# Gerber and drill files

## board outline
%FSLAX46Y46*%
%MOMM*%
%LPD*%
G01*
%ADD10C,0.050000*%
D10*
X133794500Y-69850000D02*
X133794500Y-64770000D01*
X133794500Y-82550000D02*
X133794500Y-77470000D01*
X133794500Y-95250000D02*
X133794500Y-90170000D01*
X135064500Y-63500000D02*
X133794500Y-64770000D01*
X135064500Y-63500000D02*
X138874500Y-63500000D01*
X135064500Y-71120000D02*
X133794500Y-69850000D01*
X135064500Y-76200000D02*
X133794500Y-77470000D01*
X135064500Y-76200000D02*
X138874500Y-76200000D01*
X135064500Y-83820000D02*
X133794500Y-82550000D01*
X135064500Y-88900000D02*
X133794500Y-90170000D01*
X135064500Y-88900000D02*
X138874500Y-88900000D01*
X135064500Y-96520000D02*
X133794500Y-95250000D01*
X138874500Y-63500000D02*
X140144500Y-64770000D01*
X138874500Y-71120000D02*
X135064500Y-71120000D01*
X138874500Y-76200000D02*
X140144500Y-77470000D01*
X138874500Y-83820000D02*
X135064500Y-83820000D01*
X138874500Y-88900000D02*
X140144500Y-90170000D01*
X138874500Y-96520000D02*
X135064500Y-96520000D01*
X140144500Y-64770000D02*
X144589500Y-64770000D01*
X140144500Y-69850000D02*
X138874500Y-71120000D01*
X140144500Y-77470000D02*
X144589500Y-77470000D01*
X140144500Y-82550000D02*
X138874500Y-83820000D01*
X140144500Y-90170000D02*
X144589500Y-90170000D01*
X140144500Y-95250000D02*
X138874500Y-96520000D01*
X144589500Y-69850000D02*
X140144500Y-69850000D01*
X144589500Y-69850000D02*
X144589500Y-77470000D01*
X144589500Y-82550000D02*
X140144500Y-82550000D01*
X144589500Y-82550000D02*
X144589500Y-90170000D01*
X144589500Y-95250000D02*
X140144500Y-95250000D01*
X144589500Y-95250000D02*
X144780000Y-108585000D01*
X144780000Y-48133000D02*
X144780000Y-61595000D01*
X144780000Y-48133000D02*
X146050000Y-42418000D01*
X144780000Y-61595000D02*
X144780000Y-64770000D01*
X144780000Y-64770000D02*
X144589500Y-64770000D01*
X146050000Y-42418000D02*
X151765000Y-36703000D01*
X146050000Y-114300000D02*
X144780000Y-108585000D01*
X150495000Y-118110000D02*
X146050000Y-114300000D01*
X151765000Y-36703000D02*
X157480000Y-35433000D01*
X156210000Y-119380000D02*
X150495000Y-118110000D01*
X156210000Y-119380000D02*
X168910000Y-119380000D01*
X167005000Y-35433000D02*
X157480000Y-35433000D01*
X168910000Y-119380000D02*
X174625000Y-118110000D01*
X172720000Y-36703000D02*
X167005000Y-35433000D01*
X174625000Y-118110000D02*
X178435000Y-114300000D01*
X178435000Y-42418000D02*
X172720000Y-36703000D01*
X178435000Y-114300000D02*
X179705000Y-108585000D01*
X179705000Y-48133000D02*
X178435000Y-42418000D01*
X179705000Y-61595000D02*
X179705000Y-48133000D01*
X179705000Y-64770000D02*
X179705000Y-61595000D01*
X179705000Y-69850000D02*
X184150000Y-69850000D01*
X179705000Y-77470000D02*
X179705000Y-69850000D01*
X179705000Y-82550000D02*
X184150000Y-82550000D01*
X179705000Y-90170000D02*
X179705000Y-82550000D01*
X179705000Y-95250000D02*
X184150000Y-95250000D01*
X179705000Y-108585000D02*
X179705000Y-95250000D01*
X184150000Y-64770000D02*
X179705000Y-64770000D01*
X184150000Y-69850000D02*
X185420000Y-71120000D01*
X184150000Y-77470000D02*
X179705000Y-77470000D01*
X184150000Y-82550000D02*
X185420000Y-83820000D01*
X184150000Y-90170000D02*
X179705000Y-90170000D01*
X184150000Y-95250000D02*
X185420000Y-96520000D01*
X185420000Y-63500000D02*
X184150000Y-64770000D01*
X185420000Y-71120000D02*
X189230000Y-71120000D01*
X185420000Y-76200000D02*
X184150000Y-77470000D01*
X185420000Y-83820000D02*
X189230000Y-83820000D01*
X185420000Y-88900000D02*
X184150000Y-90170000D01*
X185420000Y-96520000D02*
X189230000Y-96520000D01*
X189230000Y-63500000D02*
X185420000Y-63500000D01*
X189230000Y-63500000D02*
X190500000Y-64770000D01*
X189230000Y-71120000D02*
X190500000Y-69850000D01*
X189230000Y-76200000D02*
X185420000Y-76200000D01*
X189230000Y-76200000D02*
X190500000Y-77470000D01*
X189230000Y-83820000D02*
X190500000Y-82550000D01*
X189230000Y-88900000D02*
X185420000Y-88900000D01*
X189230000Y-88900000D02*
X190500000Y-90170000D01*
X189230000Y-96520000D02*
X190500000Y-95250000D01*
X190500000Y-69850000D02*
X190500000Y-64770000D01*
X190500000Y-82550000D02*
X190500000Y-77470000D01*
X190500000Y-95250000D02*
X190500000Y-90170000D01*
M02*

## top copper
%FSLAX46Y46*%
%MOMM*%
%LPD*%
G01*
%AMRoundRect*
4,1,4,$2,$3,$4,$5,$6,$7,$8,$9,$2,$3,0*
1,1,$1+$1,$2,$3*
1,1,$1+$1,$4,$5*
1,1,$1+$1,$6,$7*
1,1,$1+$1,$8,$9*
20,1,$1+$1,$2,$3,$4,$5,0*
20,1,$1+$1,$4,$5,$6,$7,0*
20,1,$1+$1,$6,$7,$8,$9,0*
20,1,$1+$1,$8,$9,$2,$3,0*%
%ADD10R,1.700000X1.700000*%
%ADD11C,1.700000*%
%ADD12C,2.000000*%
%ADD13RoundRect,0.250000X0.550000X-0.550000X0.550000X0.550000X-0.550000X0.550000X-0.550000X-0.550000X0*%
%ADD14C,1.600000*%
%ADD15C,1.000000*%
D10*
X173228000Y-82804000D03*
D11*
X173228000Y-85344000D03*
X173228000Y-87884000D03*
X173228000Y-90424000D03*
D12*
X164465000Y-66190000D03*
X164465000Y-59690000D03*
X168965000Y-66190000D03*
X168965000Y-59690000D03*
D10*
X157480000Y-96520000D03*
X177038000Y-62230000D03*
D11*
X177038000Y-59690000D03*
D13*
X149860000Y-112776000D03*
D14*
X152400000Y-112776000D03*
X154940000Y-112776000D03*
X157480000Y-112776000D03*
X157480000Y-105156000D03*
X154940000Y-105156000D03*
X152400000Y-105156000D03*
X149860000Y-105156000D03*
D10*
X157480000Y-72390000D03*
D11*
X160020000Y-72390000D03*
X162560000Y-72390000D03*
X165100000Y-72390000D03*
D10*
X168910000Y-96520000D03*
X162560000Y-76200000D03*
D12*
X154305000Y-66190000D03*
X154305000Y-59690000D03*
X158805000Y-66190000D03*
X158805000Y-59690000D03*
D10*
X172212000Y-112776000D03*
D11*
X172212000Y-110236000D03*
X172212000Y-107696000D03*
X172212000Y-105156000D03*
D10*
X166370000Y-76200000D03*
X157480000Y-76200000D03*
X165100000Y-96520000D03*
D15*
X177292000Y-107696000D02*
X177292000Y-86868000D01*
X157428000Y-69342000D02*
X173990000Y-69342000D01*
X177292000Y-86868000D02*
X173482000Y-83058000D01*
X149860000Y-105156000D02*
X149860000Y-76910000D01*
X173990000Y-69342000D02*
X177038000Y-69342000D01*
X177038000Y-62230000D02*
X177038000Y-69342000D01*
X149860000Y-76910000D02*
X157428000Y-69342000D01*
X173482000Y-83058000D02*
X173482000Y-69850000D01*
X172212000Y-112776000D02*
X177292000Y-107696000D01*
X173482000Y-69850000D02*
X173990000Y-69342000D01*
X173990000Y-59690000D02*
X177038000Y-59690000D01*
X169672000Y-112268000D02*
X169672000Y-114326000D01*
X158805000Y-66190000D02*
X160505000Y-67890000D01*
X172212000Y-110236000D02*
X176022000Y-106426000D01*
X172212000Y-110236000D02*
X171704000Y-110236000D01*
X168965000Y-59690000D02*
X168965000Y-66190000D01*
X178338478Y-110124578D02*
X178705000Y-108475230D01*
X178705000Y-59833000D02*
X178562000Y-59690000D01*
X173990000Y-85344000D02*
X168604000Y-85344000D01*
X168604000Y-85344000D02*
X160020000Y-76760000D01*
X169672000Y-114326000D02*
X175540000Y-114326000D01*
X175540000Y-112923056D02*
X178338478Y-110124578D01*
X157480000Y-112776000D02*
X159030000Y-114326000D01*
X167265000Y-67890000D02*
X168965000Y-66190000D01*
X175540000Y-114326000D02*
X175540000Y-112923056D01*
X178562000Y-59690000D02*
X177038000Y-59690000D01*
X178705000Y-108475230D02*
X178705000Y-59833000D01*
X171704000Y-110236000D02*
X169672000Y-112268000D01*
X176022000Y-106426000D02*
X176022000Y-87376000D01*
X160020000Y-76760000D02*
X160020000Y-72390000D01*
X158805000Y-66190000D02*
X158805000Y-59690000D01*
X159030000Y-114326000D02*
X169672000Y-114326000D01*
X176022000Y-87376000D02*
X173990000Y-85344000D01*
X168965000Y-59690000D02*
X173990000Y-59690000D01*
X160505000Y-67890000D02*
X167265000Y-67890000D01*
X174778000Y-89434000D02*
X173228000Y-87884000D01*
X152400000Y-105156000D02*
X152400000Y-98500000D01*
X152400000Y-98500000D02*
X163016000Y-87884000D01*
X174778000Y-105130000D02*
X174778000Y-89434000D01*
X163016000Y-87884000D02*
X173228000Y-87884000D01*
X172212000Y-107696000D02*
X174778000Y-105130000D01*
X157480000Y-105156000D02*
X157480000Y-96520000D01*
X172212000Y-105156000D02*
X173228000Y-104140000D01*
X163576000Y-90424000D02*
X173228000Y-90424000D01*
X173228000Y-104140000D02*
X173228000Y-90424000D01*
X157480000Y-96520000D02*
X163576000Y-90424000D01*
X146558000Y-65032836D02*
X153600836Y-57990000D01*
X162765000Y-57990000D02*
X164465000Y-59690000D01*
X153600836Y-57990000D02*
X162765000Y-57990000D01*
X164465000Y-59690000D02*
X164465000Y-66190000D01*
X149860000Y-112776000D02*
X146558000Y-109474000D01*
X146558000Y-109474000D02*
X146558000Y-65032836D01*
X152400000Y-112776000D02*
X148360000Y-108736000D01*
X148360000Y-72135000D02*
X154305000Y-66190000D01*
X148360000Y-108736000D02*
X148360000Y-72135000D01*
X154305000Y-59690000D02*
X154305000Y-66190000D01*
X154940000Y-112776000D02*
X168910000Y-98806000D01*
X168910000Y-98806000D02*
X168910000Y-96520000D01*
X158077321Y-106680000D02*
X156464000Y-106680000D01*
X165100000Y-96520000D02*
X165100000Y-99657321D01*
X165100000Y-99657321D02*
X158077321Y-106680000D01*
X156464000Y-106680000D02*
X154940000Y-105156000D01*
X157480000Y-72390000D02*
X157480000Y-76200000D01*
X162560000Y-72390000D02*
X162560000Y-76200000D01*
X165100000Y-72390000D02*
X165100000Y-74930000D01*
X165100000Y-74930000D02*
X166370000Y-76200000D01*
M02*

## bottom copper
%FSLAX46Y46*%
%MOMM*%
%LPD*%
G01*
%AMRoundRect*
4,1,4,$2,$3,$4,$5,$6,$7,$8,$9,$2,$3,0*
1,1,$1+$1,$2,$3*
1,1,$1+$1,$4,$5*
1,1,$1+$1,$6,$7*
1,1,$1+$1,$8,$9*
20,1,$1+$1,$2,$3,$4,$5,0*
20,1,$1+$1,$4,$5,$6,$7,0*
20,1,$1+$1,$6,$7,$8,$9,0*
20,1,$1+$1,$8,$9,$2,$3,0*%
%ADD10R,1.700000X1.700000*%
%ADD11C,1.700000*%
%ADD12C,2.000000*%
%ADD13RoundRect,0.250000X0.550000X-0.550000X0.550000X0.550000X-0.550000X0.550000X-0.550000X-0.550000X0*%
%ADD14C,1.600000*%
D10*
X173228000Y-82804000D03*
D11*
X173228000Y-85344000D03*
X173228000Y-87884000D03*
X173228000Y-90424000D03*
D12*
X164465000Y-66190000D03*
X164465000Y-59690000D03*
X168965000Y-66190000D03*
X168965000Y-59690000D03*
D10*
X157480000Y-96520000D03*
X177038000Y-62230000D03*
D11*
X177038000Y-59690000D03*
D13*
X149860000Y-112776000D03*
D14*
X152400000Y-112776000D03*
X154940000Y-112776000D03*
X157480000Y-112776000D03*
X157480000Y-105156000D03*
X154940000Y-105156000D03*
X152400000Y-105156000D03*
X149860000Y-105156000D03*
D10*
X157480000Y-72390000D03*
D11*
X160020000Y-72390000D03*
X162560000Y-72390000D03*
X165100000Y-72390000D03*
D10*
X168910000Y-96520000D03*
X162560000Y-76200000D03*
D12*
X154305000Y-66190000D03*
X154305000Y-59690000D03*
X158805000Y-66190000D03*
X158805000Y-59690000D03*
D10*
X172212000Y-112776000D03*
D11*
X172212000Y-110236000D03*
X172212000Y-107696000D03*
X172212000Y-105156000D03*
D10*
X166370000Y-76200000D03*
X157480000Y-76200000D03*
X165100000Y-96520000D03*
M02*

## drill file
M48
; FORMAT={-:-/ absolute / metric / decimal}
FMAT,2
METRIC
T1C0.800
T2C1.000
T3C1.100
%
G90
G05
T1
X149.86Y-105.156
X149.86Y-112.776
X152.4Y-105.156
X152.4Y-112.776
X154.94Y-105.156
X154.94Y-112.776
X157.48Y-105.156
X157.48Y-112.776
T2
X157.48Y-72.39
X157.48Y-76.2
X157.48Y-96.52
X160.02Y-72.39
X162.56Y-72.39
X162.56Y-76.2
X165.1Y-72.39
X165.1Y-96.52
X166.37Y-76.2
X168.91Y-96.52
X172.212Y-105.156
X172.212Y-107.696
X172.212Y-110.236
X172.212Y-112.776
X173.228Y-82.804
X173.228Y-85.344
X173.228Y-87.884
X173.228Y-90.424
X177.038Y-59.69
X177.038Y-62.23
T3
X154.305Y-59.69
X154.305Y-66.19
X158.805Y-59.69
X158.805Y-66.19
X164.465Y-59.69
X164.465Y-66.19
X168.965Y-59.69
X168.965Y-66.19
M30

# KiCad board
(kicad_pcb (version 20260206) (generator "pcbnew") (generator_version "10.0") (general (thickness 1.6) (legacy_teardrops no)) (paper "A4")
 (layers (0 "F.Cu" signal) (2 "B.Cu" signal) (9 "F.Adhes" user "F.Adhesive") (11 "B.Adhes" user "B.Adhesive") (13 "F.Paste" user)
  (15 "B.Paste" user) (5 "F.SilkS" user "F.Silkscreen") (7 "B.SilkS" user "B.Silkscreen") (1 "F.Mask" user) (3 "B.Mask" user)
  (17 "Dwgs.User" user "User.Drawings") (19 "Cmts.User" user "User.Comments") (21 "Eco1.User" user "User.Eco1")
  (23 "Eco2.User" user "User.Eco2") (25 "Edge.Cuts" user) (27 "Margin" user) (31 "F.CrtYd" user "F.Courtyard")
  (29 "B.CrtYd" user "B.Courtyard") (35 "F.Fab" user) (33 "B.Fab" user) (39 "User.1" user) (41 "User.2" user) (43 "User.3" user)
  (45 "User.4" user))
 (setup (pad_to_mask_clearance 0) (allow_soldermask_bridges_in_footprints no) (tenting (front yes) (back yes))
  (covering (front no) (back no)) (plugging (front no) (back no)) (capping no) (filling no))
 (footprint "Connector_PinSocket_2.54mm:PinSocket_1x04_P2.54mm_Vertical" (layer "F.Cu") (at 173.228 82.804)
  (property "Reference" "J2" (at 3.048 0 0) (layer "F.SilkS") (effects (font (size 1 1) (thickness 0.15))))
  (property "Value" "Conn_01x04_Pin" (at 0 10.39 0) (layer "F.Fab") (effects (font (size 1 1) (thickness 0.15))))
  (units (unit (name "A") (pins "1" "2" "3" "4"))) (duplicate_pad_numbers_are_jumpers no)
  (pad "1" thru_hole rect (at 0 0) (size 1.7 1.7) (drill 1) (layers "*.Cu" "*.Mask") (remove_unused_layers no) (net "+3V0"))
  (pad "2" thru_hole circle (at 0 2.54) (size 1.7 1.7) (drill 1) (layers "*.Cu" "*.Mask") (remove_unused_layers no) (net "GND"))
  (pad "3" thru_hole circle (at 0 5.08) (size 1.7 1.7) (drill 1) (layers "*.Cu" "*.Mask") (remove_unused_layers no) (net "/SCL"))
  (pad "4" thru_hole circle (at 0 7.62) (size 1.7 1.7) (drill 1) (layers "*.Cu" "*.Mask") (remove_unused_layers no) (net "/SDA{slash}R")))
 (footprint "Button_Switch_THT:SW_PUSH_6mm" (layer "F.Cu") (at 164.465 66.19 90)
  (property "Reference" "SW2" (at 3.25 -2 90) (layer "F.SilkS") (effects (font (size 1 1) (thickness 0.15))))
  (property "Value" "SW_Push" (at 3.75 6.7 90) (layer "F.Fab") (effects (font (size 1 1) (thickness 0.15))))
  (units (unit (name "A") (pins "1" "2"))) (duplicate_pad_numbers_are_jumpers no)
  (pad "1" thru_hole circle (at 0 0 180) (size 2 2) (drill 1.1) (layers "*.Cu" "*.Mask") (remove_unused_layers no) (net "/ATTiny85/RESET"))
  (pad "1" thru_hole circle (at 6.5 0 180) (size 2 2) (drill 1.1) (layers "*.Cu" "*.Mask") (remove_unused_layers no) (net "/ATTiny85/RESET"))
  (pad "2" thru_hole circle (at 0 4.5 180) (size 2 2) (drill 1.1) (layers "*.Cu" "*.Mask") (remove_unused_layers no) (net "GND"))
  (pad "2" thru_hole circle (at 6.5 4.5 180) (size 2 2) (drill 1.1) (layers "*.Cu" "*.Mask") (remove_unused_layers no) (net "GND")))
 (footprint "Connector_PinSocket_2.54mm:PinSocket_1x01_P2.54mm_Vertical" (layer "F.Cu") (at 157.48 96.52)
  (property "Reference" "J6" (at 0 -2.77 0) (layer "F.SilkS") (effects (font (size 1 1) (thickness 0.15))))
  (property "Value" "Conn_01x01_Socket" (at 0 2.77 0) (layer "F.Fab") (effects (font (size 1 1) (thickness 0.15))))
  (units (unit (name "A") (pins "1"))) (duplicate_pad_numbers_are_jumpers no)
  (pad "1" thru_hole rect (at 0 0) (size 1.7 1.7) (drill 1) (layers "*.Cu" "*.Mask") (remove_unused_layers no) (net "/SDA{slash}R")))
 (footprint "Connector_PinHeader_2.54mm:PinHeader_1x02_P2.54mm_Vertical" (layer "F.Cu") (at 177.038 62.23 180)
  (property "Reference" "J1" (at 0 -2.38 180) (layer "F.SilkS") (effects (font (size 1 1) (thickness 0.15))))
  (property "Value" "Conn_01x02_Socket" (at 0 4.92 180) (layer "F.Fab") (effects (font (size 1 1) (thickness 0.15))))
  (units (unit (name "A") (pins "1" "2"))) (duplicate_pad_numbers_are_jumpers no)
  (pad "1" thru_hole rect (at 0 0 180) (size 1.7 1.7) (drill 1) (layers "*.Cu" "*.Mask") (remove_unused_layers no) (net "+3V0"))
  (pad "2" thru_hole circle (at 0 2.54 180) (size 1.7 1.7) (drill 1) (layers "*.Cu" "*.Mask") (remove_unused_layers no) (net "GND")))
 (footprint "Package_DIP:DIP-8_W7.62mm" (layer "F.Cu") (at 149.86 112.776 90)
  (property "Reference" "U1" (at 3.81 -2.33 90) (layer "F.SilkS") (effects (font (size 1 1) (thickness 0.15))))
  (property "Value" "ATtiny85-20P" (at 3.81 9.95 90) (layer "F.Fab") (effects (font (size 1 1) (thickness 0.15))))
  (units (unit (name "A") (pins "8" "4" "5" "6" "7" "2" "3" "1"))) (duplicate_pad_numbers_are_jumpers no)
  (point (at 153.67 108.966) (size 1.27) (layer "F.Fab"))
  (pad "1" thru_hole roundrect (at 0 0 90) (size 1.6 1.6) (drill 0.8) (layers "*.Cu" "*.Mask") (remove_unused_layers no)
   (roundrect_rratio 0.15625) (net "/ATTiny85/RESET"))
  (pad "2" thru_hole circle (at 0 2.54 90) (size 1.6 1.6) (drill 0.8) (layers "*.Cu" "*.Mask") (remove_unused_layers no)
   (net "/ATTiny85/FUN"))
  (pad "3" thru_hole circle (at 0 5.08 90) (size 1.6 1.6) (drill 0.8) (layers "*.Cu" "*.Mask") (remove_unused_layers no) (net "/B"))
  (pad "4" thru_hole circle (at 0 7.62 90) (size 1.6 1.6) (drill 0.8) (layers "*.Cu" "*.Mask") (remove_unused_layers no) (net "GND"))
  (pad "5" thru_hole circle (at 7.62 7.62 90) (size 1.6 1.6) (drill 0.8) (layers "*.Cu" "*.Mask") (remove_unused_layers no)
   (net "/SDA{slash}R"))
  (pad "6" thru_hole circle (at 7.62 5.08 90) (size 1.6 1.6) (drill 0.8) (layers "*.Cu" "*.Mask") (remove_unused_layers no) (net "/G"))
  (pad "7" thru_hole circle (at 7.62 2.54 90) (size 1.6 1.6) (drill 0.8) (layers "*.Cu" "*.Mask") (remove_unused_layers no) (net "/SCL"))
  (pad "8" thru_hole circle (at 7.62 0 90) (size 1.6 1.6) (drill 0.8) (layers "*.Cu" "*.Mask") (remove_unused_layers no) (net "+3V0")))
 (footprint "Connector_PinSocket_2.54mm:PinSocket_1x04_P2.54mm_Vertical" (layer "F.Cu") (at 157.48 72.39 90)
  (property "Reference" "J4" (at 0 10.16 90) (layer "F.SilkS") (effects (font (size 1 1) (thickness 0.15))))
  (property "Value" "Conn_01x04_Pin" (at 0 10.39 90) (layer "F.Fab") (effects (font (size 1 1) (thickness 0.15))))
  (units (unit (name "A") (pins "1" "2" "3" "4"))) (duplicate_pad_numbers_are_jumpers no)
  (pad "1" thru_hole rect (at 0 0 90) (size 1.7 1.7) (drill 1) (layers "*.Cu" "*.Mask") (remove_unused_layers no) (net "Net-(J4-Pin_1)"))
  (pad "2" thru_hole circle (at 0 2.54 90) (size 1.7 1.7) (drill 1) (layers "*.Cu" "*.Mask") (remove_unused_layers no) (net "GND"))
  (pad "3" thru_hole circle (at 0 5.08 90) (size 1.7 1.7) (drill 1) (layers "*.Cu" "*.Mask") (remove_unused_layers no)
   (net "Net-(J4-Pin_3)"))
  (pad "4" thru_hole circle (at 0 7.62 90) (size 1.7 1.7) (drill 1) (layers "*.Cu" "*.Mask") (remove_unused_layers no)
   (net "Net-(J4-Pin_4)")))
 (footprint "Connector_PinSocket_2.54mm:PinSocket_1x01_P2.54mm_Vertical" (layer "F.Cu") (at 168.91 96.52)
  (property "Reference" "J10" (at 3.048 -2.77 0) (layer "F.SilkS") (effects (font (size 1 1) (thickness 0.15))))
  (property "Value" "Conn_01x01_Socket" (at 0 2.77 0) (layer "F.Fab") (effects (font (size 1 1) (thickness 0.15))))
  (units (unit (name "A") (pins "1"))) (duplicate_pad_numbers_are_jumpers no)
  (pad "1" thru_hole rect (at 0 0) (size 1.7 1.7) (drill 1) (layers "*.Cu" "*.Mask") (remove_unused_layers no) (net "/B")))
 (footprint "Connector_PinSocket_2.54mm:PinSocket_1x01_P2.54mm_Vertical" (layer "F.Cu") (at 162.56 76.2)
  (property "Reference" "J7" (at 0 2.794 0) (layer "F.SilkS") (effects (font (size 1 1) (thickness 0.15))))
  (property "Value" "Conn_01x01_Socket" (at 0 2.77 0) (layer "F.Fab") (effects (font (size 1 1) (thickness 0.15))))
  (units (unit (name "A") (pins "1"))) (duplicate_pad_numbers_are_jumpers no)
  (pad "1" thru_hole rect (at 0 0) (size 1.7 1.7) (drill 1) (layers "*.Cu" "*.Mask") (remove_unused_layers no) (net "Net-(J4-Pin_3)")))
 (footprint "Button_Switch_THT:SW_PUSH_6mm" (layer "F.Cu") (at 154.305 66.19 90)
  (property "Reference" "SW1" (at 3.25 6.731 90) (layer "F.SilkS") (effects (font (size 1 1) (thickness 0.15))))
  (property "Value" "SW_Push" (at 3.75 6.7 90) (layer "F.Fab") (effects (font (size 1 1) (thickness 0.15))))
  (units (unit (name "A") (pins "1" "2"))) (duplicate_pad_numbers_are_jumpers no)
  (pad "1" thru_hole circle (at 0 0 180) (size 2 2) (drill 1.1) (layers "*.Cu" "*.Mask") (remove_unused_layers no) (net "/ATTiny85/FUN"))
  (pad "1" thru_hole circle (at 6.5 0 180) (size 2 2) (drill 1.1) (layers "*.Cu" "*.Mask") (remove_unused_layers no) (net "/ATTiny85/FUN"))
  (pad "2" thru_hole circle (at 0 4.5 180) (size 2 2) (drill 1.1) (layers "*.Cu" "*.Mask") (remove_unused_layers no) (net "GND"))
  (pad "2" thru_hole circle (at 6.5 4.5 180) (size 2 2) (drill 1.1) (layers "*.Cu" "*.Mask") (remove_unused_layers no) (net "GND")))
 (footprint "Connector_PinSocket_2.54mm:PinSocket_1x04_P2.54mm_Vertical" (layer "F.Cu") (at 172.212 112.776 180)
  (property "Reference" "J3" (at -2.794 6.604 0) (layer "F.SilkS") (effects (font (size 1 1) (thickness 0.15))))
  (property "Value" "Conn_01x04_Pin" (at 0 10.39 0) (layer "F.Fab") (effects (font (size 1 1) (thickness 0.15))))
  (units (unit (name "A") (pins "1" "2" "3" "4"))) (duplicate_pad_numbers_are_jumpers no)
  (pad "1" thru_hole rect (at 0 0 180) (size 1.7 1.7) (drill 1) (layers "*.Cu" "*.Mask") (remove_unused_layers no) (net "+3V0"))
  (pad "2" thru_hole circle (at 0 2.54 180) (size 1.7 1.7) (drill 1) (layers "*.Cu" "*.Mask") (remove_unused_layers no) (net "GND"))
  (pad "3" thru_hole circle (at 0 5.08 180) (size 1.7 1.7) (drill 1) (layers "*.Cu" "*.Mask") (remove_unused_layers no) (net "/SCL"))
  (pad "4" thru_hole circle (at 0 7.62 180) (size 1.7 1.7) (drill 1) (layers "*.Cu" "*.Mask") (remove_unused_layers no) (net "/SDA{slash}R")))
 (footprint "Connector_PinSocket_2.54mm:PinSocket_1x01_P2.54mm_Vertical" (layer "F.Cu") (at 166.37 76.2)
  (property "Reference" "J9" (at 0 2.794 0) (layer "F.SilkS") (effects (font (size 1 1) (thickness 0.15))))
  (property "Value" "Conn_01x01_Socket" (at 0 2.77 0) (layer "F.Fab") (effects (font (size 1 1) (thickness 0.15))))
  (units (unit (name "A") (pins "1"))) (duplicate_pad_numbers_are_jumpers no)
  (pad "1" thru_hole rect (at 0 0) (size 1.7 1.7) (drill 1) (layers "*.Cu" "*.Mask") (remove_unused_layers no) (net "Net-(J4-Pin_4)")))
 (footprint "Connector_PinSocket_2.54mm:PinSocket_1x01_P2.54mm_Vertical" (layer "F.Cu") (at 157.48 76.2)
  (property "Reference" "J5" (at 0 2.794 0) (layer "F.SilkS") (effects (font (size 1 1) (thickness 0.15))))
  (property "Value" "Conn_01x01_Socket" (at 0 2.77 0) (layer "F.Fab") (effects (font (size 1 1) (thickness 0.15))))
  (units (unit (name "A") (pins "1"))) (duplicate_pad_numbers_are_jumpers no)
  (pad "1" thru_hole rect (at 0 0) (size 1.7 1.7) (drill 1) (layers "*.Cu" "*.Mask") (remove_unused_layers no) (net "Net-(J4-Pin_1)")))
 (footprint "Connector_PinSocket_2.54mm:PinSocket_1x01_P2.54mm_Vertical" (layer "F.Cu") (at 165.1 96.52)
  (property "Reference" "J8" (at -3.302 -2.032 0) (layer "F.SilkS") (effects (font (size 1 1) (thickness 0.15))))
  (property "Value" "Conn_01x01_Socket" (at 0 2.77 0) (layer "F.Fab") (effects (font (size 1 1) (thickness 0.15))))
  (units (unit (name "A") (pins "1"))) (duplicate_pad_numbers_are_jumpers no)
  (pad "1" thru_hole rect (at 0 0) (size 1.7 1.7) (drill 1) (layers "*.Cu" "*.Mask") (remove_unused_layers no) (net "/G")))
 (gr_line (start 133.7945 69.85) (end 133.7945 64.77) (stroke (width 0.05) (type default)) (layer "Edge.Cuts"))
 (gr_line (start 133.7945 82.55) (end 133.7945 77.47) (stroke (width 0.05) (type default)) (layer "Edge.Cuts"))
 (gr_line (start 133.7945 95.25) (end 133.7945 90.17) (stroke (width 0.05) (type default)) (layer "Edge.Cuts"))
 (gr_line (start 135.0645 63.5) (end 133.7945 64.77) (stroke (width 0.05) (type default)) (layer "Edge.Cuts"))
 (gr_line (start 135.0645 63.5) (end 138.8745 63.5) (stroke (width 0.05) (type default)) (layer "Edge.Cuts"))
 (gr_line (start 135.0645 71.12) (end 133.7945 69.85) (stroke (width 0.05) (type default)) (layer "Edge.Cuts"))
 (gr_line (start 135.0645 76.2) (end 133.7945 77.47) (stroke (width 0.05) (type default)) (layer "Edge.Cuts"))
 (gr_line (start 135.0645 76.2) (end 138.8745 76.2) (stroke (width 0.05) (type default)) (layer "Edge.Cuts"))
 (gr_line (start 135.0645 83.82) (end 133.7945 82.55) (stroke (width 0.05) (type default)) (layer "Edge.Cuts"))
 (gr_line (start 135.0645 88.9) (end 133.7945 90.17) (stroke (width 0.05) (type default)) (layer "Edge.Cuts"))
 (gr_line (start 135.0645 88.9) (end 138.8745 88.9) (stroke (width 0.05) (type default)) (layer "Edge.Cuts"))
 (gr_line (start 135.0645 96.52) (end 133.7945 95.25) (stroke (width 0.05) (type default)) (layer "Edge.Cuts"))
 (gr_line (start 138.8745 63.5) (end 140.1445 64.77) (stroke (width 0.05) (type default)) (layer "Edge.Cuts"))
 (gr_line (start 138.8745 71.12) (end 135.0645 71.12) (stroke (width 0.05) (type default)) (layer "Edge.Cuts"))
 (gr_line (start 138.8745 76.2) (end 140.1445 77.47) (stroke (width 0.05) (type default)) (layer "Edge.Cuts"))
 (gr_line (start 138.8745 83.82) (end 135.0645 83.82) (stroke (width 0.05) (type default)) (layer "Edge.Cuts"))
 (gr_line (start 138.8745 88.9) (end 140.1445 90.17) (stroke (width 0.05) (type default)) (layer "Edge.Cuts"))
 (gr_line (start 138.8745 96.52) (end 135.0645 96.52) (stroke (width 0.05) (type default)) (layer "Edge.Cuts"))
 (gr_line (start 140.1445 64.77) (end 144.5895 64.77) (stroke (width 0.05) (type default)) (layer "Edge.Cuts"))
 (gr_line (start 140.1445 69.85) (end 138.8745 71.12) (stroke (width 0.05) (type default)) (layer "Edge.Cuts"))
 (gr_line (start 140.1445 77.47) (end 144.5895 77.47) (stroke (width 0.05) (type default)) (layer "Edge.Cuts"))
 (gr_line (start 140.1445 82.55) (end 138.8745 83.82) (stroke (width 0.05) (type default)) (layer "Edge.Cuts"))
 (gr_line (start 140.1445 90.17) (end 144.5895 90.17) (stroke (width 0.05) (type default)) (layer "Edge.Cuts"))
 (gr_line (start 140.1445 95.25) (end 138.8745 96.52) (stroke (width 0.05) (type default)) (layer "Edge.Cuts"))
 (gr_line (start 144.5895 69.85) (end 140.1445 69.85) (stroke (width 0.05) (type default)) (layer "Edge.Cuts"))
 (gr_line (start 144.5895 69.85) (end 144.5895 77.47) (stroke (width 0.05) (type default)) (layer "Edge.Cuts"))
 (gr_line (start 144.5895 82.55) (end 140.1445 82.55) (stroke (width 0.05) (type default)) (layer "Edge.Cuts"))
 (gr_line (start 144.5895 82.55) (end 144.5895 90.17) (stroke (width 0.05) (type default)) (layer "Edge.Cuts"))
 (gr_line (start 144.5895 95.25) (end 140.1445 95.25) (stroke (width 0.05) (type default)) (layer "Edge.Cuts"))
 (gr_line (start 144.5895 95.25) (end 144.78 108.585) (stroke (width 0.05) (type default)) (layer "Edge.Cuts"))
 (gr_line (start 144.78 48.133) (end 144.78 61.595) (stroke (width 0.05) (type default)) (layer "Edge.Cuts"))
 (gr_line (start 144.78 48.133) (end 146.05 42.418) (stroke (width 0.05) (type default)) (layer "Edge.Cuts"))
 (gr_line (start 144.78 61.595) (end 144.78 64.77) (stroke (width 0.05) (type default)) (layer "Edge.Cuts"))
 (gr_line (start 144.78 64.77) (end 144.5895 64.77) (stroke (width 0.05) (type default)) (layer "Edge.Cuts"))
 (gr_line (start 146.05 42.418) (end 151.765 36.703) (stroke (width 0.05) (type default)) (layer "Edge.Cuts"))
 (gr_line (start 146.05 114.3) (end 144.78 108.585) (stroke (width 0.05) (type default)) (layer "Edge.Cuts"))
 (gr_line (start 150.495 118.11) (end 146.05 114.3) (stroke (width 0.05) (type default)) (layer "Edge.Cuts"))
 (gr_line (start 151.765 36.703) (end 157.48 35.433) (stroke (width 0.05) (type default)) (layer "Edge.Cuts"))
 (gr_line (start 156.21 119.38) (end 150.495 118.11) (stroke (width 0.05) (type default)) (layer "Edge.Cuts"))
 (gr_line (start 156.21 119.38) (end 168.91 119.38) (stroke (width 0.05) (type default)) (layer "Edge.Cuts"))
 (gr_line (start 167.005 35.433) (end 157.48 35.433) (stroke (width 0.05) (type default)) (layer "Edge.Cuts"))
 (gr_line (start 168.91 119.38) (end 174.625 118.11) (stroke (width 0.05) (type default)) (layer "Edge.Cuts"))
 (gr_line (start 172.72 36.703) (end 167.005 35.433) (stroke (width 0.05) (type default)) (layer "Edge.Cuts"))
 (gr_line (start 174.625 118.11) (end 178.435 114.3) (stroke (width 0.05) (type default)) (layer "Edge.Cuts"))
 (gr_line (start 178.435 42.418) (end 172.72 36.703) (stroke (width 0.05) (type default)) (layer "Edge.Cuts"))
 (gr_line (start 178.435 114.3) (end 179.705 108.585) (stroke (width 0.05) (type default)) (layer "Edge.Cuts"))
 (gr_line (start 179.705 48.133) (end 178.435 42.418) (stroke (width 0.05) (type default)) (layer "Edge.Cuts"))
 (gr_line (start 179.705 61.595) (end 179.705 48.133) (stroke (width 0.05) (type default)) (layer "Edge.Cuts"))
 (gr_line (start 179.705 64.77) (end 179.705 61.595) (stroke (width 0.05) (type default)) (layer "Edge.Cuts"))
 (gr_line (start 179.705 69.85) (end 184.15 69.85) (stroke (width 0.05) (type default)) (layer "Edge.Cuts"))
 (gr_line (start 179.705 77.47) (end 179.705 69.85) (stroke (width 0.05) (type default)) (layer "Edge.Cuts"))
 (gr_line (start 179.705 82.55) (end 184.15 82.55) (stroke (width 0.05) (type default)) (layer "Edge.Cuts"))
 (gr_line (start 179.705 90.17) (end 179.705 82.55) (stroke (width 0.05) (type default)) (layer "Edge.Cuts"))
 (gr_line (start 179.705 95.25) (end 184.15 95.25) (stroke (width 0.05) (type default)) (layer "Edge.Cuts"))
 (gr_line (start 179.705 108.585) (end 179.705 95.25) (stroke (width 0.05) (type default)) (layer "Edge.Cuts"))
 (gr_line (start 184.15 64.77) (end 179.705 64.77) (stroke (width 0.05) (type default)) (layer "Edge.Cuts"))
 (gr_line (start 184.15 69.85) (end 185.42 71.12) (stroke (width 0.05) (type default)) (layer "Edge.Cuts"))
 (gr_line (start 184.15 77.47) (end 179.705 77.47) (stroke (width 0.05) (type default)) (layer "Edge.Cuts"))
 (gr_line (start 184.15 82.55) (end 185.42 83.82) (stroke (width 0.05) (type default)) (layer "Edge.Cuts"))
 (gr_line (start 184.15 90.17) (end 179.705 90.17) (stroke (width 0.05) (type default)) (layer "Edge.Cuts"))
 (gr_line (start 184.15 95.25) (end 185.42 96.52) (stroke (width 0.05) (type default)) (layer "Edge.Cuts"))
 (gr_line (start 185.42 63.5) (end 184.15 64.77) (stroke (width 0.05) (type default)) (layer "Edge.Cuts"))
 (gr_line (start 185.42 71.12) (end 189.23 71.12) (stroke (width 0.05) (type default)) (layer "Edge.Cuts"))
 (gr_line (start 185.42 76.2) (end 184.15 77.47) (stroke (width 0.05) (type default)) (layer "Edge.Cuts"))
 (gr_line (start 185.42 83.82) (end 189.23 83.82) (stroke (width 0.05) (type default)) (layer "Edge.Cuts"))
 (gr_line (start 185.42 88.9) (end 184.15 90.17) (stroke (width 0.05) (type default)) (layer "Edge.Cuts"))
 (gr_line (start 185.42 96.52) (end 189.23 96.52) (stroke (width 0.05) (type default)) (layer "Edge.Cuts"))
 (gr_line (start 189.23 63.5) (end 185.42 63.5) (stroke (width 0.05) (type default)) (layer "Edge.Cuts"))
 (gr_line (start 189.23 63.5) (end 190.5 64.77) (stroke (width 0.05) (type default)) (layer "Edge.Cuts"))
 (gr_line (start 189.23 71.12) (end 190.5 69.85) (stroke (width 0.05) (type default)) (layer "Edge.Cuts"))
 (gr_line (start 189.23 76.2) (end 185.42 76.2) (stroke (width 0.05) (type default)) (layer "Edge.Cuts"))
 (gr_line (start 189.23 76.2) (end 190.5 77.47) (stroke (width 0.05) (type default)) (layer "Edge.Cuts"))
 (gr_line (start 189.23 83.82) (end 190.5 82.55) (stroke (width 0.05) (type default)) (layer "Edge.Cuts"))
 (gr_line (start 189.23 88.9) (end 185.42 88.9) (stroke (width 0.05) (type default)) (layer "Edge.Cuts"))
 (gr_line (start 189.23 88.9) (end 190.5 90.17) (stroke (width 0.05) (type default)) (layer "Edge.Cuts"))
 (gr_line (start 189.23 96.52) (end 190.5 95.25) (stroke (width 0.05) (type default)) (layer "Edge.Cuts"))
 (gr_line (start 190.5 69.85) (end 190.5 64.77) (stroke (width 0.05) (type default)) (layer "Edge.Cuts"))
 (gr_line (start 190.5 82.55) (end 190.5 77.47) (stroke (width 0.05) (type default)) (layer "Edge.Cuts"))
 (gr_line (start 190.5 95.25) (end 190.5 90.17) (stroke (width 0.05) (type default)) (layer "Edge.Cuts"))
 (segment (start 177.292 107.696) (end 177.292 86.868) (width 1) (layer "F.Cu") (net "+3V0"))
 (segment (start 157.428 69.342) (end 173.99 69.342) (width 1) (layer "F.Cu") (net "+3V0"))
 (segment (start 177.292 86.868) (end 173.482 83.058) (width 1) (layer "F.Cu") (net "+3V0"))
 (segment (start 149.86 105.156) (end 149.86 76.91) (width 1) (layer "F.Cu") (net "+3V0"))
 (segment (start 173.99 69.342) (end 177.038 69.342) (width 1) (layer "F.Cu") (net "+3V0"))
 (segment (start 177.038 62.23) (end 177.038 69.342) (width 1) (layer "F.Cu") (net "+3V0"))
 (segment (start 149.86 76.91) (end 157.428 69.342) (width 1) (layer "F.Cu") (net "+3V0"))
 (segment (start 173.482 83.058) (end 173.482 69.85) (width 1) (layer "F.Cu") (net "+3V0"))
 (segment (start 172.212 112.776) (end 177.292 107.696) (width 1) (layer "F.Cu") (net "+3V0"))
 (segment (start 173.482 69.85) (end 173.99 69.342) (width 1) (layer "F.Cu") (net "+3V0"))
 (segment (start 173.99 59.69) (end 177.038 59.69) (width 1) (layer "F.Cu") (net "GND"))
 (segment (start 169.672 112.268) (end 169.672 114.326) (width 1) (layer "F.Cu") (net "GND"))
 (segment (start 158.805 66.19) (end 160.505 67.89) (width 1) (layer "F.Cu") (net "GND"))
 (segment (start 172.212 110.236) (end 176.022 106.426) (width 1) (layer "F.Cu") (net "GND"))
 (segment (start 172.212 110.236) (end 171.704 110.236) (width 1) (layer "F.Cu") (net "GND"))
 (segment (start 168.965 59.69) (end 168.965 66.19) (width 1) (layer "F.Cu") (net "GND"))
 (segment (start 178.338478 110.124578) (end 178.705 108.47523) (width 1) (layer "F.Cu") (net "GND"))
 (segment (start 178.705 59.833) (end 178.562 59.69) (width 1) (layer "F.Cu") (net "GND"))
 (segment (start 173.99 85.344) (end 168.604 85.344) (width 1) (layer "F.Cu") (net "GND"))
 (segment (start 168.604 85.344) (end 160.02 76.76) (width 1) (layer "F.Cu") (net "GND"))
 (segment (start 169.672 114.326) (end 175.54 114.326) (width 1) (layer "F.Cu") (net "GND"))
 (segment (start 175.54 112.923056) (end 178.338478 110.124578) (width 1) (layer "F.Cu") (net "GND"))
 (segment (start 157.48 112.776) (end 159.03 114.326) (width 1) (layer "F.Cu") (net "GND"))
 (segment (start 167.265 67.89) (end 168.965 66.19) (width 1) (layer "F.Cu") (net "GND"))
 (segment (start 175.54 114.326) (end 175.54 112.923056) (width 1) (layer "F.Cu") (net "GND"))
 (segment (start 178.562 59.69) (end 177.038 59.69) (width 1) (layer "F.Cu") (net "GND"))
 (segment (start 178.705 108.47523) (end 178.705 59.833) (width 1) (layer "F.Cu") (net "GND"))
 (segment (start 171.704 110.236) (end 169.672 112.268) (width 1) (layer "F.Cu") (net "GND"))
 (segment (start 176.022 106.426) (end 176.022 87.376) (width 1) (layer "F.Cu") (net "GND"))
 (segment (start 160.02 76.76) (end 160.02 72.39) (width 1) (layer "F.Cu") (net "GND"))
 (segment (start 158.805 66.19) (end 158.805 59.69) (width 1) (layer "F.Cu") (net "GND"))
 (segment (start 159.03 114.326) (end 169.672 114.326) (width 1) (layer "F.Cu") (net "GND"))
 (segment (start 176.022 87.376) (end 173.99 85.344) (width 1) (layer "F.Cu") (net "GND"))
 (segment (start 168.965 59.69) (end 173.99 59.69) (width 1) (layer "F.Cu") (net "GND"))
 (segment (start 160.505 67.89) (end 167.265 67.89) (width 1) (layer "F.Cu") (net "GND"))
 (segment (start 174.778 89.434) (end 173.228 87.884) (width 1) (layer "F.Cu") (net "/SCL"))
 (segment (start 152.4 105.156) (end 152.4 98.5) (width 1) (layer "F.Cu") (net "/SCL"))
 (segment (start 152.4 98.5) (end 163.016 87.884) (width 1) (layer "F.Cu") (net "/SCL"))
 (segment (start 174.778 105.13) (end 174.778 89.434) (width 1) (layer "F.Cu") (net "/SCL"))
 (segment (start 163.016 87.884) (end 173.228 87.884) (width 1) (layer "F.Cu") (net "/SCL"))
 (segment (start 172.212 107.696) (end 174.778 105.13) (width 1) (layer "F.Cu") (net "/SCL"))
 (segment (start 157.48 105.156) (end 157.48 96.52) (width 1) (layer "F.Cu") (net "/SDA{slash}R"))
 (segment (start 172.212 105.156) (end 173.228 104.14) (width 1) (layer "F.Cu") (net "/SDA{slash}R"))
 (segment (start 163.576 90.424) (end 173.228 90.424) (width 1) (layer "F.Cu") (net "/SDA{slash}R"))
 (segment (start 173.228 104.14) (end 173.228 90.424) (width 1) (layer "F.Cu") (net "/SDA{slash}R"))
 (segment (start 157.48 96.52) (end 163.576 90.424) (width 1) (layer "F.Cu") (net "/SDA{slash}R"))
 (segment (start 146.558 65.032836) (end 153.600836 57.99) (width 1) (layer "F.Cu") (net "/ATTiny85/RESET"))
 (segment (start 162.765 57.99) (end 164.465 59.69) (width 1) (layer "F.Cu") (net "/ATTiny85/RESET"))
 (segment (start 153.600836 57.99) (end 162.765 57.99) (width 1) (layer "F.Cu") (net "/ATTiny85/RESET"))
 (segment (start 164.465 59.69) (end 164.465 66.19) (width 1) (layer "F.Cu") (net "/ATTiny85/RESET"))
 (segment (start 149.86 112.776) (end 146.558 109.474) (width 1) (layer "F.Cu") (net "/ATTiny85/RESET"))
 (segment (start 146.558 109.474) (end 146.558 65.032836) (width 1) (layer "F.Cu") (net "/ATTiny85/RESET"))
 (segment (start 152.4 112.776) (end 148.36 108.736) (width 1) (layer "F.Cu") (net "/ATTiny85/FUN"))
 (segment (start 148.36 72.135) (end 154.305 66.19) (width 1) (layer "F.Cu") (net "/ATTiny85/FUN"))
 (segment (start 148.36 108.736) (end 148.36 72.135) (width 1) (layer "F.Cu") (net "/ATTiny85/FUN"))
 (segment (start 154.305 59.69) (end 154.305 66.19) (width 1) (layer "F.Cu") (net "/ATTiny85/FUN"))
 (segment (start 154.94 112.776) (end 168.91 98.806) (width 1) (layer "F.Cu") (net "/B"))
 (segment (start 168.91 98.806) (end 168.91 96.52) (width 1) (layer "F.Cu") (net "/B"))
 (segment (start 158.077321 106.68) (end 156.464 106.68) (width 1) (layer "F.Cu") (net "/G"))
 (segment (start 165.1 96.52) (end 165.1 99.657321) (width 1) (layer "F.Cu") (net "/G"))
 (segment (start 165.1 99.657321) (end 158.077321 106.68) (width 1) (layer "F.Cu") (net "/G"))
 (segment (start 156.464 106.68) (end 154.94 105.156) (width 1) (layer "F.Cu") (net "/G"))
 (segment (start 157.48 72.39) (end 157.48 76.2) (width 1) (layer "F.Cu") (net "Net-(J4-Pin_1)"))
 (segment (start 162.56 72.39) (end 162.56 76.2) (width 1) (layer "F.Cu") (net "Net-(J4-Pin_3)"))
 (segment (start 165.1 72.39) (end 165.1 74.93) (width 1) (layer "F.Cu") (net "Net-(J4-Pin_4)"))
 (segment (start 165.1 74.93) (end 166.37 76.2) (width 1) (layer "F.Cu") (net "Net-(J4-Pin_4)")))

